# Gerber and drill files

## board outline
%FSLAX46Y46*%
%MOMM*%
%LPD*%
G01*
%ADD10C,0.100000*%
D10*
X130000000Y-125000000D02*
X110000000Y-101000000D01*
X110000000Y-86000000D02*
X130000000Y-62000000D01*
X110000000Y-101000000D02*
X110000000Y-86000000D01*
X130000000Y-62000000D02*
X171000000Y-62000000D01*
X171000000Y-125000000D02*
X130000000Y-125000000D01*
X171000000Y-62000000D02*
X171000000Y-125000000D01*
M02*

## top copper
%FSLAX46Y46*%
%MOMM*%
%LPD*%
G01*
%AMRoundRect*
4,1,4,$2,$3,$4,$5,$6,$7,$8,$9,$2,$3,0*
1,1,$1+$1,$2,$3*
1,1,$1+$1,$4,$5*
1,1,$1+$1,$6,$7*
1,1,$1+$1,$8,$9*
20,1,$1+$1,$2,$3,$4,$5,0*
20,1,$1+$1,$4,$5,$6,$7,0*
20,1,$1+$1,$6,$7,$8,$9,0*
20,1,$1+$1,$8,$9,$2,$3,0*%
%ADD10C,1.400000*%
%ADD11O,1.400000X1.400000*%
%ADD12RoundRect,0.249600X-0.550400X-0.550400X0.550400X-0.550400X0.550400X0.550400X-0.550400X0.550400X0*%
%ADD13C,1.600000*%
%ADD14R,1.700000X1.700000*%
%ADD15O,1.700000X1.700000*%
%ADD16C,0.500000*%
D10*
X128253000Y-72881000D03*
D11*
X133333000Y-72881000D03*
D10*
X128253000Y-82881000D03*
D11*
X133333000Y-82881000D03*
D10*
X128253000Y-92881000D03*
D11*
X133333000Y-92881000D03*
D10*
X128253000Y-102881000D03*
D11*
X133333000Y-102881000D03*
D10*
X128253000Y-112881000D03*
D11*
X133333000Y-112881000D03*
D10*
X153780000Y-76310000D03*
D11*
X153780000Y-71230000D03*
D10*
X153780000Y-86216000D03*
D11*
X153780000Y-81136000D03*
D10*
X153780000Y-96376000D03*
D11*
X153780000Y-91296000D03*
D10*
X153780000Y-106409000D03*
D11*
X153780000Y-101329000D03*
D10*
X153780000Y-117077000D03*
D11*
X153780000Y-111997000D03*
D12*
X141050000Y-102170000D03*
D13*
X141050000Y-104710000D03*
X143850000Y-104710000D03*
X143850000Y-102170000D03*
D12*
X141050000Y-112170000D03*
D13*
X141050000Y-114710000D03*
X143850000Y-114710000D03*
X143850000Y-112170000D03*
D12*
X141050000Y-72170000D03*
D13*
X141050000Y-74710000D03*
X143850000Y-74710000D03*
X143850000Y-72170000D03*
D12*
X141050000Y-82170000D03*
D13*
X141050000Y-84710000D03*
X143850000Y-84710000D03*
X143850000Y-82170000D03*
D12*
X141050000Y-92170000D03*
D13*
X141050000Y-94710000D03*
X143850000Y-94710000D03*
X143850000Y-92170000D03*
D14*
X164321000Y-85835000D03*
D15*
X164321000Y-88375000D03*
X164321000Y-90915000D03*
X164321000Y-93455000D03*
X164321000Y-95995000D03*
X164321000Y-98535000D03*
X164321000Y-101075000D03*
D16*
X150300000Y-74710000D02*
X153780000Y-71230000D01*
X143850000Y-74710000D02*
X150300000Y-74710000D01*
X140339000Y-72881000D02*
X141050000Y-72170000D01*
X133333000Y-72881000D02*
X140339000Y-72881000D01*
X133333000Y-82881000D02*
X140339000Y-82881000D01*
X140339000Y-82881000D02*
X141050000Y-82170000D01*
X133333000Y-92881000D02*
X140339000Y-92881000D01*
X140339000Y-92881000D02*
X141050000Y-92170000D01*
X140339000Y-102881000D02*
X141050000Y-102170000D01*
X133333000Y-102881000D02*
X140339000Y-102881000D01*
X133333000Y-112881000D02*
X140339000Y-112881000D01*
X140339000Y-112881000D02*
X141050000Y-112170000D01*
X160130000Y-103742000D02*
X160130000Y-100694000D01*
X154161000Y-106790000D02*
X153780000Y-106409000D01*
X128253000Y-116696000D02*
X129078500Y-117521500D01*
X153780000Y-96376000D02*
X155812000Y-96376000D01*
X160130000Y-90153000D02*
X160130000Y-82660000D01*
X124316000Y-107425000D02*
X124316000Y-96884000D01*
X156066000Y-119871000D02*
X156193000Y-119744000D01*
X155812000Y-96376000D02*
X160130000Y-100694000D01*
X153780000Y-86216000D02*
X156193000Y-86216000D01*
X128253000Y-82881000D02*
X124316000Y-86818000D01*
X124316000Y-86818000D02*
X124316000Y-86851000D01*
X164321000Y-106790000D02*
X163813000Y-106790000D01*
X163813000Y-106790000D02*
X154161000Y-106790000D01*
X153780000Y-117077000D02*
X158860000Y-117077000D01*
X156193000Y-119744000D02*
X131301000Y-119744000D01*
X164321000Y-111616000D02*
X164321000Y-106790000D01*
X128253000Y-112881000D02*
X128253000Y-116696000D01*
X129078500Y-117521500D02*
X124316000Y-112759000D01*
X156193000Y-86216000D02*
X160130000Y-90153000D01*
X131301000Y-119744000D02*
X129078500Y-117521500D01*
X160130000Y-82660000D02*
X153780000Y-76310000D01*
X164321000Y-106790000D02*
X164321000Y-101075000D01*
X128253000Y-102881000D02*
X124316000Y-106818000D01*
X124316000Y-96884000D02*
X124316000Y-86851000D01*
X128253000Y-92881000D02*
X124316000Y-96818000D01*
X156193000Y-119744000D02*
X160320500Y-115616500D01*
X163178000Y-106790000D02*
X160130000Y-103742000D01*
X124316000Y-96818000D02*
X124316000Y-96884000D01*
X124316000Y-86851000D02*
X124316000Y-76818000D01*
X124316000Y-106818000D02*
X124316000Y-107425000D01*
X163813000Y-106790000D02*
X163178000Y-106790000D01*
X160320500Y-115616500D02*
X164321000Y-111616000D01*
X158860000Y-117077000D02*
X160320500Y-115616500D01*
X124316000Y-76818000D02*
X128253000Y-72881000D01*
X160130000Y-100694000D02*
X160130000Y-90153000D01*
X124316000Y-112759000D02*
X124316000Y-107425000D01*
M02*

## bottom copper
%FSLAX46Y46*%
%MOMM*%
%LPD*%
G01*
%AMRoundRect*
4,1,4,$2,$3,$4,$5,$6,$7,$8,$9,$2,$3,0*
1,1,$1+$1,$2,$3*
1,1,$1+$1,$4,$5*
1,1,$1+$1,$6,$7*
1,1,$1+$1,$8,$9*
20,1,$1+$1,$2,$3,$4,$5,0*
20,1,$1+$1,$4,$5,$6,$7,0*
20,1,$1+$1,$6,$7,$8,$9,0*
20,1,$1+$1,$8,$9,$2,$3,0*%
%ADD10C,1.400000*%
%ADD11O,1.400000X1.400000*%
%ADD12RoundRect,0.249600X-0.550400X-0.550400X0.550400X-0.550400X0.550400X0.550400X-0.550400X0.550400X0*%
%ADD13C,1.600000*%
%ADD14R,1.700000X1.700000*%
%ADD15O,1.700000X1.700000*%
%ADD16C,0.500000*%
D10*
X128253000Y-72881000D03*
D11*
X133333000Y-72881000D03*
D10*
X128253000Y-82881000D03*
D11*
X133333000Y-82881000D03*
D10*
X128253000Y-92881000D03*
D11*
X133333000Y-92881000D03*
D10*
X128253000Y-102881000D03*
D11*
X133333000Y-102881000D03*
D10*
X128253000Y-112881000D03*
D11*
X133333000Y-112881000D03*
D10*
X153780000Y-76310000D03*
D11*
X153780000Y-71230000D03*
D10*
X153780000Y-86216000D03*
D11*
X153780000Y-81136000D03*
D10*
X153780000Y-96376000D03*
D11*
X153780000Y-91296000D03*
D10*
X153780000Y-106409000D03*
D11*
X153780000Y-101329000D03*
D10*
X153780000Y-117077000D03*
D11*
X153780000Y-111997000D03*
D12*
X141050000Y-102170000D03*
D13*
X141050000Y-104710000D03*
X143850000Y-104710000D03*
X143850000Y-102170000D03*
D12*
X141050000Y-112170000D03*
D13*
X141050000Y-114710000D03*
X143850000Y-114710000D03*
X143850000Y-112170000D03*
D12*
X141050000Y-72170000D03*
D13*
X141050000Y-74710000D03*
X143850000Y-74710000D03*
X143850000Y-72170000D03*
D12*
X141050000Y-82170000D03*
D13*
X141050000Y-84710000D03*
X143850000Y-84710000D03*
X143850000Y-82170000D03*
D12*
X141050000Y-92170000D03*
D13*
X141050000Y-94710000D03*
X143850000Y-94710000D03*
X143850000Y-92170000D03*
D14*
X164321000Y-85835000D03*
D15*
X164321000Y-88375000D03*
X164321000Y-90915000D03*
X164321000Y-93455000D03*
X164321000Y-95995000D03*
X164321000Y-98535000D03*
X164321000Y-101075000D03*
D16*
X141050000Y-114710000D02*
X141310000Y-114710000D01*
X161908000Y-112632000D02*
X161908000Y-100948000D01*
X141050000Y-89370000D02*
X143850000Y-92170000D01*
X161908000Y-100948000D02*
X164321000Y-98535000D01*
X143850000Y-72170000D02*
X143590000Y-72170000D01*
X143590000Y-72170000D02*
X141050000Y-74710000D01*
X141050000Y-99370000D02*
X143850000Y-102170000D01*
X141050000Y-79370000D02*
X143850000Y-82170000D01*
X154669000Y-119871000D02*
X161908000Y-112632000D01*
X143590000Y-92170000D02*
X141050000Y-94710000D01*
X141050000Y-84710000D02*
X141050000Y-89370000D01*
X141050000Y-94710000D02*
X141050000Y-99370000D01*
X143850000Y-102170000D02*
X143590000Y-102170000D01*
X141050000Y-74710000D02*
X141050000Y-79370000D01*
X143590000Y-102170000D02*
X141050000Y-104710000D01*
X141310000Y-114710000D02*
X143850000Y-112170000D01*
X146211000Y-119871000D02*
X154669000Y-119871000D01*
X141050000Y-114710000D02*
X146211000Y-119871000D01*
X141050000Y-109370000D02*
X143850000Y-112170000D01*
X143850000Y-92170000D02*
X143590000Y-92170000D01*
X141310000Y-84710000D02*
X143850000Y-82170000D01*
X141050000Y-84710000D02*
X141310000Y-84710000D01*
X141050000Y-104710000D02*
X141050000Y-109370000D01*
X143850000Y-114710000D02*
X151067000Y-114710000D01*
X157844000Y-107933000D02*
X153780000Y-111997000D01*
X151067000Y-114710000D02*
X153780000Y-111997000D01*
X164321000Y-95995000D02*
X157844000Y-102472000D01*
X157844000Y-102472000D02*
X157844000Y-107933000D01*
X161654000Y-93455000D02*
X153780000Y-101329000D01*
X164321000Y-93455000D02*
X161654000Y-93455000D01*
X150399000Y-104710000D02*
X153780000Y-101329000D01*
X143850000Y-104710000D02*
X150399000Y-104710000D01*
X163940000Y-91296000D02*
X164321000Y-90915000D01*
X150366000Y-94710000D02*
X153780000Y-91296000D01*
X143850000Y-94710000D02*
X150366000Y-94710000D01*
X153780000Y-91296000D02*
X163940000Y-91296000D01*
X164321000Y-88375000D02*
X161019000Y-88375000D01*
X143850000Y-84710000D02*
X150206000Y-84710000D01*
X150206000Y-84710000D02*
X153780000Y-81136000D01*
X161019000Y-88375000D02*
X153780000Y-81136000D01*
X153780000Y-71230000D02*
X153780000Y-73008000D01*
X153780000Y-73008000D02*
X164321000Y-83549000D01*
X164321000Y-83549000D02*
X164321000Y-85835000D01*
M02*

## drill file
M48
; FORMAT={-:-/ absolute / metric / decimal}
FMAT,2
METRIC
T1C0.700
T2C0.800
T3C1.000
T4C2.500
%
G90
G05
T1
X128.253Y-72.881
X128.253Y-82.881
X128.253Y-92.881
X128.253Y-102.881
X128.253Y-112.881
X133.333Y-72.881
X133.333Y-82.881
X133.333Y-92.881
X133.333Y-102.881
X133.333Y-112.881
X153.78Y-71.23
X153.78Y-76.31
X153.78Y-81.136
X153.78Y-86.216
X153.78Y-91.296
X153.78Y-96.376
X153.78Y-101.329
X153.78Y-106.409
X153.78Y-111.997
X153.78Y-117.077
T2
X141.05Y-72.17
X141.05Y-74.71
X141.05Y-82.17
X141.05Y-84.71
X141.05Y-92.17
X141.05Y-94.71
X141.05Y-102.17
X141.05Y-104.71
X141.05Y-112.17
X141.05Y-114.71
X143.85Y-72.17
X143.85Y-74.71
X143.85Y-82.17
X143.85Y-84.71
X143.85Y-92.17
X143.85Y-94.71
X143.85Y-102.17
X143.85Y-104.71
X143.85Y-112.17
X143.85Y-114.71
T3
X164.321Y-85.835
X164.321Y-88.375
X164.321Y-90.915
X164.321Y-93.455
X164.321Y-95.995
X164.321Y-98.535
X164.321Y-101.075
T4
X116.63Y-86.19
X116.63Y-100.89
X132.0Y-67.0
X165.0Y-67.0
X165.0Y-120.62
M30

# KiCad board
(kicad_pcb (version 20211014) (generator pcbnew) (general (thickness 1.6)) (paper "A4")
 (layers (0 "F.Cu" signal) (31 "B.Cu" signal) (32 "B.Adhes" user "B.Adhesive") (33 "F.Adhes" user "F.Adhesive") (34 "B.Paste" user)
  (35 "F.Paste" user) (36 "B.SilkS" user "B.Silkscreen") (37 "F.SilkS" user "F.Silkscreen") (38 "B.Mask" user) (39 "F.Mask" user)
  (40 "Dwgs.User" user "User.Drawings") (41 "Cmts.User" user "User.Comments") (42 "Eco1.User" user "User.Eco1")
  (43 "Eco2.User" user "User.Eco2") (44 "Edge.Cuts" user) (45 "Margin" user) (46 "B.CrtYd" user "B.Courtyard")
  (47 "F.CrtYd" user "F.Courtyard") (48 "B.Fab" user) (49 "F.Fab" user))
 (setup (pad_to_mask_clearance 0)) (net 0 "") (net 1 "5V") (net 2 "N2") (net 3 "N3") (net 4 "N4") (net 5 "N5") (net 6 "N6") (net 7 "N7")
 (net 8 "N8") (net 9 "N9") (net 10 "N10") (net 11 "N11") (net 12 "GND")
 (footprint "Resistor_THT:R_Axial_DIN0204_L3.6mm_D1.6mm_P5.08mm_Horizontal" (layer "F.Cu") (at 128.253 72.881)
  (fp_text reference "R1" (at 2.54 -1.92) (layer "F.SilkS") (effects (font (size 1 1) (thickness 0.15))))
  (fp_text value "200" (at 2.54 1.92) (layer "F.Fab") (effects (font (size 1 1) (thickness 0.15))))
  (pad "1" thru_hole circle locked (at 0 0) (size 1.4 1.4) (drill 0.7) (layers *.Cu *.Mask) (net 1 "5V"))
  (pad "2" thru_hole oval locked (at 5.08 0) (size 1.4 1.4) (drill 0.7) (layers *.Cu *.Mask) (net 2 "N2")))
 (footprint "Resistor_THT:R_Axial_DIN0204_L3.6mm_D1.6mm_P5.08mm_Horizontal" (layer "F.Cu") (at 128.253 82.881)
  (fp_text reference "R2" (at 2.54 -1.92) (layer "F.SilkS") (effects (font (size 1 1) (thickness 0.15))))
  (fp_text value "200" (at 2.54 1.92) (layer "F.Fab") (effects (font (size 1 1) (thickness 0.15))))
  (pad "1" thru_hole circle locked (at 0 0) (size 1.4 1.4) (drill 0.7) (layers *.Cu *.Mask) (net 1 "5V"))
  (pad "2" thru_hole oval locked (at 5.08 0) (size 1.4 1.4) (drill 0.7) (layers *.Cu *.Mask) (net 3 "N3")))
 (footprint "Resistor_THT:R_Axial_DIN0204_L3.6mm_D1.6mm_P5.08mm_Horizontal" (layer "F.Cu") (at 128.253 92.881)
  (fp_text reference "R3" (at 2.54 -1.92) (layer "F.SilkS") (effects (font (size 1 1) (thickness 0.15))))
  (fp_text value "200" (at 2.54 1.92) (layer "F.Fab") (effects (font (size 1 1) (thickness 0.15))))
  (pad "1" thru_hole circle locked (at 0 0) (size 1.4 1.4) (drill 0.7) (layers *.Cu *.Mask) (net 1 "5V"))
  (pad "2" thru_hole oval locked (at 5.08 0) (size 1.4 1.4) (drill 0.7) (layers *.Cu *.Mask) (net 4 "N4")))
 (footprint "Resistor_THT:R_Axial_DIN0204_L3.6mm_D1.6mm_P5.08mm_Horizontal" (layer "F.Cu") (at 128.253 102.881)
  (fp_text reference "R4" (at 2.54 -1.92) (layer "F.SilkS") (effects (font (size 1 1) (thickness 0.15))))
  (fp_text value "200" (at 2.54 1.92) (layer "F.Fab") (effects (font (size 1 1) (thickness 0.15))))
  (pad "1" thru_hole circle locked (at 0 0) (size 1.4 1.4) (drill 0.7) (layers *.Cu *.Mask) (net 1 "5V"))
  (pad "2" thru_hole oval locked (at 5.08 0) (size 1.4 1.4) (drill 0.7) (layers *.Cu *.Mask) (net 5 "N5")))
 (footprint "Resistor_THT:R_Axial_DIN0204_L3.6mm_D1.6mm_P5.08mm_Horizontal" (layer "F.Cu") (at 128.253 112.881)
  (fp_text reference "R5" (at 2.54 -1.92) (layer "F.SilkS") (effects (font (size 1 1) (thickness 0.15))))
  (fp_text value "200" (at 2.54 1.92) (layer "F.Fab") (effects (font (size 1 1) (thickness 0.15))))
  (pad "1" thru_hole circle locked (at 0 0) (size 1.4 1.4) (drill 0.7) (layers *.Cu *.Mask) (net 1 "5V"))
  (pad "2" thru_hole oval locked (at 5.08 0) (size 1.4 1.4) (drill 0.7) (layers *.Cu *.Mask) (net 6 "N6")))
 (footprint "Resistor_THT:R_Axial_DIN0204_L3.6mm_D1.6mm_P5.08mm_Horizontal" (layer "F.Cu") (at 153.78 76.31 90)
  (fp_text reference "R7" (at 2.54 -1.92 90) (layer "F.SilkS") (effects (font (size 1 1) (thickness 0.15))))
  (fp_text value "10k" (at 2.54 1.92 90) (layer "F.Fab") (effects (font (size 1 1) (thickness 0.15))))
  (pad "1" thru_hole circle locked (at 0 0 90) (size 1.4 1.4) (drill 0.7) (layers *.Cu *.Mask) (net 1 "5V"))
  (pad "2" thru_hole oval locked (at 5.08 0 90) (size 1.4 1.4) (drill 0.7) (layers *.Cu *.Mask) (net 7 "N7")))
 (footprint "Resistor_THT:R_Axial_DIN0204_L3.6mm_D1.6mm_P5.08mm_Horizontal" (layer "F.Cu") (at 153.78 86.216 90)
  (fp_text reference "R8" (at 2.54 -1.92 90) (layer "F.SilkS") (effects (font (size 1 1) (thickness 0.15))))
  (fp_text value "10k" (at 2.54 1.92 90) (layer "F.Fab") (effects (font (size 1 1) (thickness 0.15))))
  (pad "1" thru_hole circle locked (at 0 0 90) (size 1.4 1.4) (drill 0.7) (layers *.Cu *.Mask) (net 1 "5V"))
  (pad "2" thru_hole oval locked (at 5.08 0 90) (size 1.4 1.4) (drill 0.7) (layers *.Cu *.Mask) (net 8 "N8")))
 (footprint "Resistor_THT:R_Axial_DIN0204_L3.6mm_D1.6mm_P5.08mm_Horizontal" (layer "F.Cu") (at 153.78 96.376 90)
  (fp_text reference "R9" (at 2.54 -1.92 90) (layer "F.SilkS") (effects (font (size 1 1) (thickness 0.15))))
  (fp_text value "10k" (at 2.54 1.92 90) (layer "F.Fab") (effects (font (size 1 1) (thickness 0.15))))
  (pad "1" thru_hole circle locked (at 0 0 90) (size 1.4 1.4) (drill 0.7) (layers *.Cu *.Mask) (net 1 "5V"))
  (pad "2" thru_hole oval locked (at 5.08 0 90) (size 1.4 1.4) (drill 0.7) (layers *.Cu *.Mask) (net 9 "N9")))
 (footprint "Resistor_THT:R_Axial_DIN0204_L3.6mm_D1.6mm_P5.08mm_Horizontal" (layer "F.Cu") (at 153.78 106.409 90)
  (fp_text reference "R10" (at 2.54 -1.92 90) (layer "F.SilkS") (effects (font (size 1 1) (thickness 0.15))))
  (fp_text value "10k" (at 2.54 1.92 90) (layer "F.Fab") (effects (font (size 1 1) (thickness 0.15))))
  (pad "1" thru_hole circle locked (at 0 0 90) (size 1.4 1.4) (drill 0.7) (layers *.Cu *.Mask) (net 1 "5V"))
  (pad "2" thru_hole oval locked (at 5.08 0 90) (size 1.4 1.4) (drill 0.7) (layers *.Cu *.Mask) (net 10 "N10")))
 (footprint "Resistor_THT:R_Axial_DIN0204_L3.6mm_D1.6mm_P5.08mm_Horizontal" (layer "F.Cu") (at 153.78 117.077 90)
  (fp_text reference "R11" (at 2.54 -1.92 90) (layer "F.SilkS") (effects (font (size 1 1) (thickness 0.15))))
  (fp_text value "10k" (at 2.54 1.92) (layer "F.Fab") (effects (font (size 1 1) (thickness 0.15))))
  (pad "1" thru_hole circle locked (at 0 0 90) (size 1.4 1.4) (drill 0.7) (layers *.Cu *.Mask) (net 1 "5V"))
  (pad "2" thru_hole oval locked (at 5.08 0 90) (size 1.4 1.4) (drill 0.7) (layers *.Cu *.Mask) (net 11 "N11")))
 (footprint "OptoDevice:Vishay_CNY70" (layer "F.Cu") (at 141.05 102.17)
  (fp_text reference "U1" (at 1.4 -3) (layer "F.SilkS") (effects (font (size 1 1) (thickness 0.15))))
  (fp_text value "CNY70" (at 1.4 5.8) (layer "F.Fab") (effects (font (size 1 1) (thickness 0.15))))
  (pad "1" thru_hole roundrect locked (at 0 0) (size 1.6 1.6) (drill 0.8) (layers *.Cu *.Mask) (roundrect_rratio 0.156) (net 5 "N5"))
  (pad "2" thru_hole circle locked (at 0 2.54) (size 1.6 1.6) (drill 0.8) (layers *.Cu *.Mask) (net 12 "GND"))
  (pad "3" thru_hole circle locked (at 2.8 2.54) (size 1.6 1.6) (drill 0.8) (layers *.Cu *.Mask) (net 10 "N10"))
  (pad "4" thru_hole circle locked (at 2.8 0) (size 1.6 1.6) (drill 0.8) (layers *.Cu *.Mask) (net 12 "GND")))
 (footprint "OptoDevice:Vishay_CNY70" (layer "F.Cu") (at 141.05 112.17)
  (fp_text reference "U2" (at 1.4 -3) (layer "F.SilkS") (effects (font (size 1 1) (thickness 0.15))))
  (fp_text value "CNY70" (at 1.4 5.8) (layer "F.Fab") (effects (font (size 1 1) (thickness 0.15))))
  (pad "1" thru_hole roundrect locked (at 0 0) (size 1.6 1.6) (drill 0.8) (layers *.Cu *.Mask) (roundrect_rratio 0.156) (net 6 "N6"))
  (pad "2" thru_hole circle locked (at 0 2.54) (size 1.6 1.6) (drill 0.8) (layers *.Cu *.Mask) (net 12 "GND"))
  (pad "3" thru_hole circle locked (at 2.8 2.54) (size 1.6 1.6) (drill 0.8) (layers *.Cu *.Mask) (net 11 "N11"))
  (pad "4" thru_hole circle locked (at 2.8 0) (size 1.6 1.6) (drill 0.8) (layers *.Cu *.Mask) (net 12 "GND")))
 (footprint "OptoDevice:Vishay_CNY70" (layer "F.Cu") (at 141.05 72.17)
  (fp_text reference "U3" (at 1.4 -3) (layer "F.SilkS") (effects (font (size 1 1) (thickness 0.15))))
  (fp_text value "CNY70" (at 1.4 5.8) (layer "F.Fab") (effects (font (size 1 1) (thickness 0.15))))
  (pad "1" thru_hole roundrect locked (at 0 0) (size 1.6 1.6) (drill 0.8) (layers *.Cu *.Mask) (roundrect_rratio 0.156) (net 2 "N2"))
  (pad "2" thru_hole circle locked (at 0 2.54) (size 1.6 1.6) (drill 0.8) (layers *.Cu *.Mask) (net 12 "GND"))
  (pad "3" thru_hole circle locked (at 2.8 2.54) (size 1.6 1.6) (drill 0.8) (layers *.Cu *.Mask) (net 7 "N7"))
  (pad "4" thru_hole circle locked (at 2.8 0) (size 1.6 1.6) (drill 0.8) (layers *.Cu *.Mask) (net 12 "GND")))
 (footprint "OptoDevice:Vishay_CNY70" (layer "F.Cu") (at 141.05 82.17)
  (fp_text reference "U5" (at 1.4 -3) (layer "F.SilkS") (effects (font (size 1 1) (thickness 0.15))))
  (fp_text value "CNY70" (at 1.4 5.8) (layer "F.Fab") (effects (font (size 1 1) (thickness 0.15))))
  (pad "1" thru_hole roundrect locked (at 0 0) (size 1.6 1.6) (drill 0.8) (layers *.Cu *.Mask) (roundrect_rratio 0.156) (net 3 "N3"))
  (pad "2" thru_hole circle locked (at 0 2.54) (size 1.6 1.6) (drill 0.8) (layers *.Cu *.Mask) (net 12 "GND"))
  (pad "3" thru_hole circle locked (at 2.8 2.54) (size 1.6 1.6) (drill 0.8) (layers *.Cu *.Mask) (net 8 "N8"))
  (pad "4" thru_hole circle locked (at 2.8 0) (size 1.6 1.6) (drill 0.8) (layers *.Cu *.Mask) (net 12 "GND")))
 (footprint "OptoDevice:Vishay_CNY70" (layer "F.Cu") (at 141.05 92.17)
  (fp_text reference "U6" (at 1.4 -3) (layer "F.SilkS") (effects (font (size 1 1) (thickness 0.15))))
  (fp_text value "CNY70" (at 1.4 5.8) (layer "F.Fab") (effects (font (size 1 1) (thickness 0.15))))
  (pad "1" thru_hole roundrect locked (at 0 0) (size 1.6 1.6) (drill 0.8) (layers *.Cu *.Mask) (roundrect_rratio 0.156) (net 4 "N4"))
  (pad "2" thru_hole circle locked (at 0 2.54) (size 1.6 1.6) (drill 0.8) (layers *.Cu *.Mask) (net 12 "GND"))
  (pad "3" thru_hole circle locked (at 2.8 2.54) (size 1.6 1.6) (drill 0.8) (layers *.Cu *.Mask) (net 9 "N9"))
  (pad "4" thru_hole circle locked (at 2.8 0) (size 1.6 1.6) (drill 0.8) (layers *.Cu *.Mask) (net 12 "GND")))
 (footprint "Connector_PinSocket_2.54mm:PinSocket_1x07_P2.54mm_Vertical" (layer "F.Cu") (at 164.321 85.835)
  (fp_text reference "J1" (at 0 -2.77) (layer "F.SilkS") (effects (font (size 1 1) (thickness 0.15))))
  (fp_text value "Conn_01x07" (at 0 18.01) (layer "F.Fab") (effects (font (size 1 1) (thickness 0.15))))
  (pad "1" thru_hole rect locked (at 0 0) (size 1.7 1.7) (drill 1) (layers *.Cu *.Mask) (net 7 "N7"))
  (pad "2" thru_hole oval locked (at 0 2.54) (size 1.7 1.7) (drill 1) (layers *.Cu *.Mask) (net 8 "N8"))
  (pad "3" thru_hole oval locked (at 0 5.08) (size 1.7 1.7) (drill 1) (layers *.Cu *.Mask) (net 9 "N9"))
  (pad "4" thru_hole oval locked (at 0 7.62) (size 1.7 1.7) (drill 1) (layers *.Cu *.Mask) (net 10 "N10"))
  (pad "5" thru_hole oval locked (at 0 10.16) (size 1.7 1.7) (drill 1) (layers *.Cu *.Mask) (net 11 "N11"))
  (pad "6" thru_hole oval locked (at 0 12.7) (size 1.7 1.7) (drill 1) (layers *.Cu *.Mask) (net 12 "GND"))
  (pad "7" thru_hole oval locked (at 0 15.24) (size 1.7 1.7) (drill 1) (layers *.Cu *.Mask) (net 1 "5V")))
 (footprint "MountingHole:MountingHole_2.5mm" (layer "F.Cu") (at 116.63 86.19)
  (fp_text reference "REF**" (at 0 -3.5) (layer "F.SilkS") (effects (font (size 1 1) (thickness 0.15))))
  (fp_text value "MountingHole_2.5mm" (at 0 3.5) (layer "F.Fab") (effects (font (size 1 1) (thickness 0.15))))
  (pad "" np_thru_hole circle (at 0 0) (size 2.5 2.5) (drill 2.5) (layers *.Cu *.Mask)))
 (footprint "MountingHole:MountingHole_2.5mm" (layer "F.Cu") (at 132 67)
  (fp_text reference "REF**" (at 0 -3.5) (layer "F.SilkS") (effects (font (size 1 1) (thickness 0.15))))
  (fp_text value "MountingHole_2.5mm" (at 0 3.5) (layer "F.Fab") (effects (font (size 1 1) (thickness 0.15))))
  (pad "" np_thru_hole circle (at 0 0) (size 2.5 2.5) (drill 2.5) (layers *.Cu *.Mask)))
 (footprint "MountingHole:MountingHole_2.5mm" (layer "F.Cu") (at 165 67)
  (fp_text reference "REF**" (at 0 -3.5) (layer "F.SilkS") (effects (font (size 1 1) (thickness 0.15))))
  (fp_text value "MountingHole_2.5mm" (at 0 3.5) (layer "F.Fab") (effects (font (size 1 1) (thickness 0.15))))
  (pad "" np_thru_hole circle (at 0 0) (size 2.5 2.5) (drill 2.5) (layers *.Cu *.Mask)))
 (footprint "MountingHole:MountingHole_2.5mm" (layer "F.Cu") (at 116.63 100.89)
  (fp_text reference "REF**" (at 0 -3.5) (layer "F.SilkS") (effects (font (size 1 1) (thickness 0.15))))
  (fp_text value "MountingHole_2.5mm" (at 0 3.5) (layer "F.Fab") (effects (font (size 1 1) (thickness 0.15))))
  (pad "" np_thru_hole circle (at 0 0) (size 2.5 2.5) (drill 2.5) (layers *.Cu *.Mask)))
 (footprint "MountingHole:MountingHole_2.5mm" (layer "F.Cu") (at 165 120.62)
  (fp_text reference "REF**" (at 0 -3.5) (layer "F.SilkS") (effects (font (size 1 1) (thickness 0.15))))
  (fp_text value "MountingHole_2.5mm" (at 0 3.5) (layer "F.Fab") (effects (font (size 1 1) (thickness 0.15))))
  (pad "" np_thru_hole circle (at 0 0) (size 2.5 2.5) (drill 2.5) (layers *.Cu *.Mask)))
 (gr_line (start 130 125) (end 110 101) (layer "Edge.Cuts") (width 0.1))
 (gr_line (start 110 86) (end 130 62) (layer "Edge.Cuts") (width 0.1))
 (gr_line (start 110 101) (end 110 86) (layer "Edge.Cuts") (width 0.1))
 (gr_line (start 130 62) (end 171 62) (layer "Edge.Cuts") (width 0.1))
 (gr_line (start 171 125) (end 130 125) (layer "Edge.Cuts") (width 0.1))
 (gr_line (start 171 62) (end 171 125) (layer "Edge.Cuts") (width 0.1))
 (segment (start 141.05 114.71) (end 141.31 114.71) (width 0.5) (layer "B.Cu") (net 12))
 (segment (start 161.908 112.632) (end 161.908 100.948) (width 0.5) (layer "B.Cu") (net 12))
 (segment (start 141.05 89.37) (end 143.85 92.17) (width 0.5) (layer "B.Cu") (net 12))
 (segment (start 161.908 100.948) (end 164.321 98.535) (width 0.5) (layer "B.Cu") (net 12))
 (segment (start 143.85 72.17) (end 143.59 72.17) (width 0.5) (layer "B.Cu") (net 12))
 (segment (start 143.59 72.17) (end 141.05 74.71) (width 0.5) (layer "B.Cu") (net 12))
 (segment (start 141.05 99.37) (end 143.85 102.17) (width 0.5) (layer "B.Cu") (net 12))
 (segment (start 141.05 79.37) (end 143.85 82.17) (width 0.5) (layer "B.Cu") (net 12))
 (segment (start 154.669 119.871) (end 161.908 112.632) (width 0.5) (layer "B.Cu") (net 12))
 (segment (start 143.59 92.17) (end 141.05 94.71) (width 0.5) (layer "B.Cu") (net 12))
 (segment (start 141.05 84.71) (end 141.05 89.37) (width 0.5) (layer "B.Cu") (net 12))
 (segment (start 141.05 94.71) (end 141.05 99.37) (width 0.5) (layer "B.Cu") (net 12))
 (segment (start 143.85 102.17) (end 143.59 102.17) (width 0.5) (layer "B.Cu") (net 12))
 (segment (start 141.05 74.71) (end 141.05 79.37) (width 0.5) (layer "B.Cu") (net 12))
 (segment (start 143.59 102.17) (end 141.05 104.71) (width 0.5) (layer "B.Cu") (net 12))
 (segment (start 141.31 114.71) (end 143.85 112.17) (width 0.5) (layer "B.Cu") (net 12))
 (segment (start 146.211 119.871) (end 154.669 119.871) (width 0.5) (layer "B.Cu") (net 12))
 (segment (start 141.05 114.71) (end 146.211 119.871) (width 0.5) (layer "B.Cu") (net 12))
 (segment (start 141.05 109.37) (end 143.85 112.17) (width 0.5) (layer "B.Cu") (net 12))
 (segment (start 143.85 92.17) (end 143.59 92.17) (width 0.5) (layer "B.Cu") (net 12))
 (segment (start 141.31 84.71) (end 143.85 82.17) (width 0.5) (layer "B.Cu") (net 12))
 (segment (start 141.05 84.71) (end 141.31 84.71) (width 0.5) (layer "B.Cu") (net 12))
 (segment (start 141.05 104.71) (end 141.05 109.37) (width 0.5) (layer "B.Cu") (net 12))
 (segment (start 143.85 114.71) (end 151.067 114.71) (width 0.5) (layer "B.Cu") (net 11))
 (segment (start 157.844 107.933) (end 153.78 111.997) (width 0.5) (layer "B.Cu") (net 11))
 (segment (start 151.067 114.71) (end 153.78 111.997) (width 0.5) (layer "B.Cu") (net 11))
 (segment (start 164.321 95.995) (end 157.844 102.472) (width 0.5) (layer "B.Cu") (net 11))
 (segment (start 157.844 102.472) (end 157.844 107.933) (width 0.5) (layer "B.Cu") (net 11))
 (segment (start 161.654 93.455) (end 153.78 101.329) (width 0.5) (layer "B.Cu") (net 10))
 (segment (start 164.321 93.455) (end 161.654 93.455) (width 0.5) (layer "B.Cu") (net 10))
 (segment (start 150.399 104.71) (end 153.78 101.329) (width 0.5) (layer "B.Cu") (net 10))
 (segment (start 143.85 104.71) (end 150.399 104.71) (width 0.5) (layer "B.Cu") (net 10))
 (segment (start 163.94 91.296) (end 164.321 90.915) (width 0.5) (layer "B.Cu") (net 9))
 (segment (start 150.366 94.71) (end 153.78 91.296) (width 0.5) (layer "B.Cu") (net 9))
 (segment (start 143.85 94.71) (end 150.366 94.71) (width 0.5) (layer "B.Cu") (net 9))
 (segment (start 153.78 91.296) (end 163.94 91.296) (width 0.5) (layer "B.Cu") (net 9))
 (segment (start 164.321 88.375) (end 161.019 88.375) (width 0.5) (layer "B.Cu") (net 8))
 (segment (start 143.85 84.71) (end 150.206 84.71) (width 0.5) (layer "B.Cu") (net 8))
 (segment (start 150.206 84.71) (end 153.78 81.136) (width 0.5) (layer "B.Cu") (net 8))
 (segment (start 161.019 88.375) (end 153.78 81.136) (width 0.5) (layer "B.Cu") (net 8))
 (segment (start 150.3 74.71) (end 153.78 71.23) (width 0.5) (layer "F.Cu") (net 7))
 (segment (start 143.85 74.71) (end 150.3 74.71) (width 0.5) (layer "F.Cu") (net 7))
 (segment (start 153.78 71.23) (end 153.78 73.008) (width 0.5) (layer "B.Cu") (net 7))
 (segment (start 153.78 73.008) (end 164.321 83.549) (width 0.5) (layer "B.Cu") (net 7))
 (segment (start 164.321 83.549) (end 164.321 85.835) (width 0.5) (layer "B.Cu") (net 7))
 (segment (start 140.339 72.881) (end 141.05 72.17) (width 0.5) (layer "F.Cu") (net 2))
 (segment (start 133.333 72.881) (end 140.339 72.881) (width 0.5) (layer "F.Cu") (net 2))
 (segment (start 133.333 82.881) (end 140.339 82.881) (width 0.5) (layer "F.Cu") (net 3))
 (segment (start 140.339 82.881) (end 141.05 82.17) (width 0.5) (layer "F.Cu") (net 3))
 (segment (start 133.333 92.881) (end 140.339 92.881) (width 0.5) (layer "F.Cu") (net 4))
 (segment (start 140.339 92.881) (end 141.05 92.17) (width 0.5) (layer "F.Cu") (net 4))
 (segment (start 140.339 102.881) (end 141.05 102.17) (width 0.5) (layer "F.Cu") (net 5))
 (segment (start 133.333 102.881) (end 140.339 102.881) (width 0.5) (layer "F.Cu") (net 5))
 (segment (start 133.333 112.881) (end 140.339 112.881) (width 0.5) (layer "F.Cu") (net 6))
 (segment (start 140.339 112.881) (end 141.05 112.17) (width 0.5) (layer "F.Cu") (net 6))
 (segment (start 160.13 103.742) (end 160.13 100.694) (width 0.5) (layer "F.Cu") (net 1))
 (segment (start 154.161 106.79) (end 153.78 106.409) (width 0.5) (layer "F.Cu") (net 1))
 (segment (start 128.253 116.696) (end 129.0785 117.5215) (width 0.5) (layer "F.Cu") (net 1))
 (segment (start 153.78 96.376) (end 155.812 96.376) (width 0.5) (layer "F.Cu") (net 1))
 (segment (start 160.13 90.153) (end 160.13 82.66) (width 0.5) (layer "F.Cu") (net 1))
 (segment (start 124.316 107.425) (end 124.316 96.884) (width 0.5) (layer "F.Cu") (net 1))
 (segment (start 156.066 119.871) (end 156.193 119.744) (width 0.5) (layer "F.Cu") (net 1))
 (segment (start 155.812 96.376) (end 160.13 100.694) (width 0.5) (layer "F.Cu") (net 1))
 (segment (start 153.78 86.216) (end 156.193 86.216) (width 0.5) (layer "F.Cu") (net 1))
 (segment (start 128.253 82.881) (end 124.316 86.818) (width 0.5) (layer "F.Cu") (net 1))
 (segment (start 124.316 86.818) (end 124.316 86.851) (width 0.5) (layer "F.Cu") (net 1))
 (segment (start 164.321 106.79) (end 163.813 106.79) (width 0.5) (layer "F.Cu") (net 1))
 (segment (start 163.813 106.79) (end 154.161 106.79) (width 0.5) (layer "F.Cu") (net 1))
 (segment (start 153.78 117.077) (end 158.86 117.077) (width 0.5) (layer "F.Cu") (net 1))
 (segment (start 156.193 119.744) (end 131.301 119.744) (width 0.5) (layer "F.Cu") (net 1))
 (segment (start 164.321 111.616) (end 164.321 106.79) (width 0.5) (layer "F.Cu") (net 1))
 (segment (start 128.253 112.881) (end 128.253 116.696) (width 0.5) (layer "F.Cu") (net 1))
 (segment (start 129.0785 117.5215) (end 124.316 112.759) (width 0.5) (layer "F.Cu") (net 1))
 (segment (start 156.193 86.216) (end 160.13 90.153) (width 0.5) (layer "F.Cu") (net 1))
 (segment (start 131.301 119.744) (end 129.0785 117.5215) (width 0.5) (layer "F.Cu") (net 1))
 (segment (start 160.13 82.66) (end 153.78 76.31) (width 0.5) (layer "F.Cu") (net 1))
 (segment (start 164.321 106.79) (end 164.321 101.075) (width 0.5) (layer "F.Cu") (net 1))
 (segment (start 128.253 102.881) (end 124.316 106.818) (width 0.5) (layer "F.Cu") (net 1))
 (segment (start 124.316 96.884) (end 124.316 86.851) (width 0.5) (layer "F.Cu") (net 1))
 (segment (start 128.253 92.881) (end 124.316 96.818) (width 0.5) (layer "F.Cu") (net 1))
 (segment (start 156.193 119.744) (end 160.3205 115.6165) (width 0.5) (layer "F.Cu") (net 1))
 (segment (start 163.178 106.79) (end 160.13 103.742) (width 0.5) (layer "F.Cu") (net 1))
 (segment (start 124.316 96.818) (end 124.316 96.884) (width 0.5) (layer "F.Cu") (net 1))
 (segment (start 124.316 86.851) (end 124.316 76.818) (width 0.5) (layer "F.Cu") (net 1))
 (segment (start 124.316 106.818) (end 124.316 107.425) (width 0.5) (layer "F.Cu") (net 1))
 (segment (start 163.813 106.79) (end 163.178 106.79) (width 0.5) (layer "F.Cu") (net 1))
 (segment (start 160.3205 115.6165) (end 164.321 111.616) (width 0.5) (layer "F.Cu") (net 1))
 (segment (start 158.86 117.077) (end 160.3205 115.6165) (width 0.5) (layer "F.Cu") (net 1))
 (segment (start 124.316 76.818) (end 128.253 72.881) (width 0.5) (layer "F.Cu") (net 1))
 (segment (start 160.13 100.694) (end 160.13 90.153) (width 0.5) (layer "F.Cu") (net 1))
 (segment (start 124.316 112.759) (end 124.316 107.425) (width 0.5) (layer "F.Cu") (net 1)))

